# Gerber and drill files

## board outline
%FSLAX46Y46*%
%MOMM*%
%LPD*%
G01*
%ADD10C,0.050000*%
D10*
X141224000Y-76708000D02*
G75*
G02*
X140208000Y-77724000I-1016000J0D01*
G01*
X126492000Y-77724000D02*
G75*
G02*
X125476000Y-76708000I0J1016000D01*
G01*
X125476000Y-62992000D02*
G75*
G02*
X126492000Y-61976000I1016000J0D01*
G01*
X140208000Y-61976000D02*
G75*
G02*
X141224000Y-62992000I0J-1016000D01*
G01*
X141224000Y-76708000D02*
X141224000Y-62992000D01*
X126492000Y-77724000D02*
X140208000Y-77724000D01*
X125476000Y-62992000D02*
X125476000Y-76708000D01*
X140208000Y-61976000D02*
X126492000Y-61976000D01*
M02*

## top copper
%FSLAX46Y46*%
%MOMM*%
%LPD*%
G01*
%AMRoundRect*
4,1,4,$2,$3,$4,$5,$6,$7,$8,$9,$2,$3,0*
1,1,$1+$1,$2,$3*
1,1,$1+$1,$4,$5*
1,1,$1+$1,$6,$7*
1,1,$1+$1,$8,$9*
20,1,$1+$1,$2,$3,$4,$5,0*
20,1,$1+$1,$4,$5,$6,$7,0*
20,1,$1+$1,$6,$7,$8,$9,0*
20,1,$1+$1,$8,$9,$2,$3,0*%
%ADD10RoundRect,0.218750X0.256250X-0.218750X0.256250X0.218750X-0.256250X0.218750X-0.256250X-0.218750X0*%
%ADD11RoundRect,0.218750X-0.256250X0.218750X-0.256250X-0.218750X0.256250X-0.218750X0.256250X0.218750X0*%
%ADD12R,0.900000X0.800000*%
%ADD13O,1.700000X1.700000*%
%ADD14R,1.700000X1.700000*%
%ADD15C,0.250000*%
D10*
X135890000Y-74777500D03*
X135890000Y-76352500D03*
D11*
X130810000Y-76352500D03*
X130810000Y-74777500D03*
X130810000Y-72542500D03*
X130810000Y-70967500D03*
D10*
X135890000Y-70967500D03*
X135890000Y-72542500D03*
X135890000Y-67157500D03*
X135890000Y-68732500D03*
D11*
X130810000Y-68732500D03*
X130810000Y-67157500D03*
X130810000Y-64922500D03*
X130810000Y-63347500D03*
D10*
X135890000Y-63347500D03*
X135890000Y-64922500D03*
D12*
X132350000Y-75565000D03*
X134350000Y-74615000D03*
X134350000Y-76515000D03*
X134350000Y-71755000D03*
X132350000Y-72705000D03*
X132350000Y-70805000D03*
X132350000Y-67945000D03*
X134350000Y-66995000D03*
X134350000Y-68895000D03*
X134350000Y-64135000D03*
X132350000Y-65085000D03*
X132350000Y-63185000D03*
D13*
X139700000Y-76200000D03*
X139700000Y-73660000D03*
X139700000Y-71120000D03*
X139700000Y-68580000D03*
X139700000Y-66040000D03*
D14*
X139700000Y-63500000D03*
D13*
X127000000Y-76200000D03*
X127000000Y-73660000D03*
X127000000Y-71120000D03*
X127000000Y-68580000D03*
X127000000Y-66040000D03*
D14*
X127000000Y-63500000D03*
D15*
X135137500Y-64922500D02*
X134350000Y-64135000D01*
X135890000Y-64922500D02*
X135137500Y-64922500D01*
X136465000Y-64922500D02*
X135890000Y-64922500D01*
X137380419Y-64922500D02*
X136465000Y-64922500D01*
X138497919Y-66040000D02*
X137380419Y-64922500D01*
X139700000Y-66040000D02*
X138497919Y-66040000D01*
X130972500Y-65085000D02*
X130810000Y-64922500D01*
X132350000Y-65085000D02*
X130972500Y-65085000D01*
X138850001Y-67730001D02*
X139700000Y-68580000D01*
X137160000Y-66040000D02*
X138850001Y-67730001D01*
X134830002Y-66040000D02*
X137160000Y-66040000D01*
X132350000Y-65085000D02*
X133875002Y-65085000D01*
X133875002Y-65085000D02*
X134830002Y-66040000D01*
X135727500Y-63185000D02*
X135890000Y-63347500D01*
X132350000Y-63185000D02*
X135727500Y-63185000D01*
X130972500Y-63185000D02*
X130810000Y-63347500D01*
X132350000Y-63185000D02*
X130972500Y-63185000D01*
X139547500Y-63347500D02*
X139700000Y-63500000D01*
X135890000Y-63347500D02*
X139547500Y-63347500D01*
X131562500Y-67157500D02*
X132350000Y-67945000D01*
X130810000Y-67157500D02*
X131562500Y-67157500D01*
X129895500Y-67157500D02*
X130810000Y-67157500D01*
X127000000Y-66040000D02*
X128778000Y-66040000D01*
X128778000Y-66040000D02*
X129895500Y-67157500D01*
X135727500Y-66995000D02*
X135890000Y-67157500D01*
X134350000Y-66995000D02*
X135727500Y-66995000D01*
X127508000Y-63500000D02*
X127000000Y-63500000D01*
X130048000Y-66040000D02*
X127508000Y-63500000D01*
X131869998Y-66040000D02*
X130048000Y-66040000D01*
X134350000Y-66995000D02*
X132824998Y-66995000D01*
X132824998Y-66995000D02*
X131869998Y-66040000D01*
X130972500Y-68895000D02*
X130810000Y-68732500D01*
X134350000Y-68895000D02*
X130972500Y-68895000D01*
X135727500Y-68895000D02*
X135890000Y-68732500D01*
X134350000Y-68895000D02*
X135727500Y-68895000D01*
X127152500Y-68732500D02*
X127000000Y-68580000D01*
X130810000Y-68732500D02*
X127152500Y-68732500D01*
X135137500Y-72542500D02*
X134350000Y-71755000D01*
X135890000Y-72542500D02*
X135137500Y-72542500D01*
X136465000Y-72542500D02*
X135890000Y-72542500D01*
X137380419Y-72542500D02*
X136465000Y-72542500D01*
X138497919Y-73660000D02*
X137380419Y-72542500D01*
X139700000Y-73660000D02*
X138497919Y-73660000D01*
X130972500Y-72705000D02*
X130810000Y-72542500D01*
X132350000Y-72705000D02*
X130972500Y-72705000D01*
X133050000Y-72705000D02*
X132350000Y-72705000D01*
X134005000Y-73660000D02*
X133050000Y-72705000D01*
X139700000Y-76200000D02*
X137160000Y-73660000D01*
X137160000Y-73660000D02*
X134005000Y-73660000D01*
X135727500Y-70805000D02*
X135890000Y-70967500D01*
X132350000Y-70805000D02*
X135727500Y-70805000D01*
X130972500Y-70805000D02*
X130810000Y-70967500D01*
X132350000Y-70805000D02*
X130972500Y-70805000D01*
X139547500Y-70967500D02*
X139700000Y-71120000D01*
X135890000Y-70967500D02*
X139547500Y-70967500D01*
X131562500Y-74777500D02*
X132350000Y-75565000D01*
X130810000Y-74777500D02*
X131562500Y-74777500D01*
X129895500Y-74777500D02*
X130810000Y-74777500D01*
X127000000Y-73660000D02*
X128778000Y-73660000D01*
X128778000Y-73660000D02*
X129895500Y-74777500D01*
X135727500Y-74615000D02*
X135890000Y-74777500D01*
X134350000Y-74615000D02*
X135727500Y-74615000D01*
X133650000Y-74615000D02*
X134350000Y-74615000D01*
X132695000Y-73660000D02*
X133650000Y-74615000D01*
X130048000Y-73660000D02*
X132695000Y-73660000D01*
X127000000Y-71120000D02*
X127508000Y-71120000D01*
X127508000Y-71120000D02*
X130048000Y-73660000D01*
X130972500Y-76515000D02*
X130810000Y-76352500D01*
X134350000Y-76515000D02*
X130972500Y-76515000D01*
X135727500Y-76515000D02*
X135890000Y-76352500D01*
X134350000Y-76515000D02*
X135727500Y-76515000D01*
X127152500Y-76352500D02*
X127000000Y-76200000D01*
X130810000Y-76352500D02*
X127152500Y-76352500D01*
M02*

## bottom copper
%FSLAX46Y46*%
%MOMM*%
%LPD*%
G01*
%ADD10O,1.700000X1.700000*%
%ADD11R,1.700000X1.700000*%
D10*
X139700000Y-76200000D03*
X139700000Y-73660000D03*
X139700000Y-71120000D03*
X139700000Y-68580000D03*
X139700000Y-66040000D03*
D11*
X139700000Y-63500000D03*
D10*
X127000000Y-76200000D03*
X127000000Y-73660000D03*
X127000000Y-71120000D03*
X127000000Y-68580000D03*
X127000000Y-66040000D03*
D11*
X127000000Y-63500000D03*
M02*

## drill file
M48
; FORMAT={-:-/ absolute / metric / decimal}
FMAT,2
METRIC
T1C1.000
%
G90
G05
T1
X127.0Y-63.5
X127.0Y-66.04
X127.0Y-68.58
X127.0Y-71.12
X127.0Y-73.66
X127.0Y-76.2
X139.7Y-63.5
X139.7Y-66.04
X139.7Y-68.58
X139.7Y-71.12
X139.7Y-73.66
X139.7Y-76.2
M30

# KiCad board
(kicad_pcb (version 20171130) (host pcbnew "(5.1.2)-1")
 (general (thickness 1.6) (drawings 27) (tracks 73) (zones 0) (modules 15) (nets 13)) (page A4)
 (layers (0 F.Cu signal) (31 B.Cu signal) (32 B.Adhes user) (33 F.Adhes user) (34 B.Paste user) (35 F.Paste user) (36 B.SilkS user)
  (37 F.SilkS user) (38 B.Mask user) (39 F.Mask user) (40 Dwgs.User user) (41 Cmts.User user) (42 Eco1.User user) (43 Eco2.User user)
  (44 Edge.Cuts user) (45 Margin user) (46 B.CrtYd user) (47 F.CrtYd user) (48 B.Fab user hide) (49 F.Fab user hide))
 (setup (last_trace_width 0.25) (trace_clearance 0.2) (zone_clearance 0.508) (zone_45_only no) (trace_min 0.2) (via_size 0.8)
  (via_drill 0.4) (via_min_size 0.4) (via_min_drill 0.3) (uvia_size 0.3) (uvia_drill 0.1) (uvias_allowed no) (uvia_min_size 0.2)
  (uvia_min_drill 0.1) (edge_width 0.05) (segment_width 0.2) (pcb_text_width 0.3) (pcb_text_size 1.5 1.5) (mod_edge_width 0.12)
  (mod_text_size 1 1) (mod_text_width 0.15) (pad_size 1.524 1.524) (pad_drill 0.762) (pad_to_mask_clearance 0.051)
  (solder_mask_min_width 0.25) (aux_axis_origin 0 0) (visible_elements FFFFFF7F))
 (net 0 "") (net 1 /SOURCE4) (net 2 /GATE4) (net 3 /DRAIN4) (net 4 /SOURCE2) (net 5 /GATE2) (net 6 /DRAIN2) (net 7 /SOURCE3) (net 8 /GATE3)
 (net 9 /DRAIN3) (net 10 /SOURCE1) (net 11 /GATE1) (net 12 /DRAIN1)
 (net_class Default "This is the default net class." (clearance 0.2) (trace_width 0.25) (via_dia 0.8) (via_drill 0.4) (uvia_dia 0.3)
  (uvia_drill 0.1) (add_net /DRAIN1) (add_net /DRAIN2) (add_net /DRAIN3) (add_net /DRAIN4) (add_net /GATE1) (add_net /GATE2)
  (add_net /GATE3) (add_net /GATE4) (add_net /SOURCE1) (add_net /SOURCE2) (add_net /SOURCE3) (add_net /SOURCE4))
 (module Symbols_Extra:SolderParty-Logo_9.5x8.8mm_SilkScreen (layer B.Cu) (at 133.35 73.406 180)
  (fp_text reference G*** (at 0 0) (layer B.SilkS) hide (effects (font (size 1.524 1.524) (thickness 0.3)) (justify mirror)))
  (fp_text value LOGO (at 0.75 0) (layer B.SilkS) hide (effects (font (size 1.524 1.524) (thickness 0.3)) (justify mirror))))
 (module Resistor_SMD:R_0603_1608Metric (layer F.Cu) (at 135.89 75.565 90)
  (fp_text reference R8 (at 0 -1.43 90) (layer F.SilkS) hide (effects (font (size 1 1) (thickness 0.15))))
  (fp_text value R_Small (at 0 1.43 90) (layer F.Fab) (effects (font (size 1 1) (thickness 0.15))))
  (pad 2 smd roundrect (at 0.7875 0 90) (size 0.875 0.95) (layers F.Cu F.Paste F.Mask) (roundrect_rratio 0.25) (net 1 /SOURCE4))
  (pad 1 smd roundrect (at -0.7875 0 90) (size 0.875 0.95) (layers F.Cu F.Paste F.Mask) (roundrect_rratio 0.25) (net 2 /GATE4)))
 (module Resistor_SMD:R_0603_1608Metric (layer F.Cu) (at 130.81 75.565 270)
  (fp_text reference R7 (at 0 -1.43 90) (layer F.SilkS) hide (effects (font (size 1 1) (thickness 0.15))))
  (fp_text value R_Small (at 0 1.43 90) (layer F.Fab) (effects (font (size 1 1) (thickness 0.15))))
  (pad 2 smd roundrect (at 0.7875 0 270) (size 0.875 0.95) (layers F.Cu F.Paste F.Mask) (roundrect_rratio 0.25) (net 2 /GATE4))
  (pad 1 smd roundrect (at -0.7875 0 270) (size 0.875 0.95) (layers F.Cu F.Paste F.Mask) (roundrect_rratio 0.25) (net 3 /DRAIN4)))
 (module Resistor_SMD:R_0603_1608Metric (layer F.Cu) (at 130.81 71.755 270)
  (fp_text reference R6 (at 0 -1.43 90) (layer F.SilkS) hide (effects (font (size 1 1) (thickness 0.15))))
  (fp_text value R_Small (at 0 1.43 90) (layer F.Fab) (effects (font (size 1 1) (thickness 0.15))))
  (pad 2 smd roundrect (at 0.7875 0 270) (size 0.875 0.95) (layers F.Cu F.Paste F.Mask) (roundrect_rratio 0.25) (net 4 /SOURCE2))
  (pad 1 smd roundrect (at -0.7875 0 270) (size 0.875 0.95) (layers F.Cu F.Paste F.Mask) (roundrect_rratio 0.25) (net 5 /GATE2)))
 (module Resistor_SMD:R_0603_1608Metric (layer F.Cu) (at 135.89 71.755 90)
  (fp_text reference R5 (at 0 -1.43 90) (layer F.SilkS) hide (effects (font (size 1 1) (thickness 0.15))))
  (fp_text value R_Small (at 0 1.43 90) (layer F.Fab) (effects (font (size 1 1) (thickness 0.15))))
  (pad 2 smd roundrect (at 0.7875 0 90) (size 0.875 0.95) (layers F.Cu F.Paste F.Mask) (roundrect_rratio 0.25) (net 5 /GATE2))
  (pad 1 smd roundrect (at -0.7875 0 90) (size 0.875 0.95) (layers F.Cu F.Paste F.Mask) (roundrect_rratio 0.25) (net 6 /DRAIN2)))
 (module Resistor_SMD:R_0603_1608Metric (layer F.Cu) (at 135.89 67.945 90)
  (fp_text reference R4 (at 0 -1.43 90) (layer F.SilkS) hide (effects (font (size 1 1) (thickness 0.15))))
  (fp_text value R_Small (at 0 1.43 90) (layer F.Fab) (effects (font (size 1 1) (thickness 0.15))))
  (pad 2 smd roundrect (at 0.7875 0 90) (size 0.875 0.95) (layers F.Cu F.Paste F.Mask) (roundrect_rratio 0.25) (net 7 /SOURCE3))
  (pad 1 smd roundrect (at -0.7875 0 90) (size 0.875 0.95) (layers F.Cu F.Paste F.Mask) (roundrect_rratio 0.25) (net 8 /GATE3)))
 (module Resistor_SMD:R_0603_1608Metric (layer F.Cu) (at 130.81 67.945 270)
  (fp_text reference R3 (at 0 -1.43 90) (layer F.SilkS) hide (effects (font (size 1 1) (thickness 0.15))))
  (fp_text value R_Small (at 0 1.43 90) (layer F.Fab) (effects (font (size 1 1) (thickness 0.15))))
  (pad 2 smd roundrect (at 0.7875 0 270) (size 0.875 0.95) (layers F.Cu F.Paste F.Mask) (roundrect_rratio 0.25) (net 8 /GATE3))
  (pad 1 smd roundrect (at -0.7875 0 270) (size 0.875 0.95) (layers F.Cu F.Paste F.Mask) (roundrect_rratio 0.25) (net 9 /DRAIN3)))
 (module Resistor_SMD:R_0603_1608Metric (layer F.Cu) (at 130.81 64.135 270)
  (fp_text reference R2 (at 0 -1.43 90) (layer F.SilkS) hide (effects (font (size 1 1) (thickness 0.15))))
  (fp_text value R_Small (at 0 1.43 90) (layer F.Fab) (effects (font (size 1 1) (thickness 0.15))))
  (pad 2 smd roundrect (at 0.7875 0 270) (size 0.875 0.95) (layers F.Cu F.Paste F.Mask) (roundrect_rratio 0.25) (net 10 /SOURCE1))
  (pad 1 smd roundrect (at -0.7875 0 270) (size 0.875 0.95) (layers F.Cu F.Paste F.Mask) (roundrect_rratio 0.25) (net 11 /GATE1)))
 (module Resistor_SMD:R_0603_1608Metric (layer F.Cu) (at 135.89 64.135 90)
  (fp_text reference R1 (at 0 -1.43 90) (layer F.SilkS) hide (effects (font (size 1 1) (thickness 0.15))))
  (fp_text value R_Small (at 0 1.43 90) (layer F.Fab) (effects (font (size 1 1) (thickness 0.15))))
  (pad 2 smd roundrect (at 0.7875 0 90) (size 0.875 0.95) (layers F.Cu F.Paste F.Mask) (roundrect_rratio 0.25) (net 11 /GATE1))
  (pad 1 smd roundrect (at -0.7875 0 90) (size 0.875 0.95) (layers F.Cu F.Paste F.Mask) (roundrect_rratio 0.25) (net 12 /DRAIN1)))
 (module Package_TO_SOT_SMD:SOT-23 (layer F.Cu) (at 133.35 75.565 180)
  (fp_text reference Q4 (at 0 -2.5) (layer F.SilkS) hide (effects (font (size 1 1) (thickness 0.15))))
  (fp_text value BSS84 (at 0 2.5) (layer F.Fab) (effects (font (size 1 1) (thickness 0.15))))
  (pad 3 smd rect (at 1 0 180) (size 0.9 0.8) (layers F.Cu F.Paste F.Mask) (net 3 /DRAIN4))
  (pad 2 smd rect (at -1 0.95 180) (size 0.9 0.8) (layers F.Cu F.Paste F.Mask) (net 1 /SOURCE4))
  (pad 1 smd rect (at -1 -0.95 180) (size 0.9 0.8) (layers F.Cu F.Paste F.Mask) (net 2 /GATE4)))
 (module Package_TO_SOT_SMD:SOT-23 (layer F.Cu) (at 133.35 71.755)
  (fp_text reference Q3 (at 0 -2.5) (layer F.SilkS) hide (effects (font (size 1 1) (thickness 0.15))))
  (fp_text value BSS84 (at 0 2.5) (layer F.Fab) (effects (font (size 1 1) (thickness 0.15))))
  (pad 3 smd rect (at 1 0) (size 0.9 0.8) (layers F.Cu F.Paste F.Mask) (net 6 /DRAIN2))
  (pad 2 smd rect (at -1 0.95) (size 0.9 0.8) (layers F.Cu F.Paste F.Mask) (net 4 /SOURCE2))
  (pad 1 smd rect (at -1 -0.95) (size 0.9 0.8) (layers F.Cu F.Paste F.Mask) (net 5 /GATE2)))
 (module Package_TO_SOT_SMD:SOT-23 (layer F.Cu) (at 133.35 67.945 180)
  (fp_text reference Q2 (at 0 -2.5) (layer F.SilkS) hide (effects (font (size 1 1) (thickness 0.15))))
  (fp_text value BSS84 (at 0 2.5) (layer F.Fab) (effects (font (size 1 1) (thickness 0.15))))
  (pad 3 smd rect (at 1 0 180) (size 0.9 0.8) (layers F.Cu F.Paste F.Mask) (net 9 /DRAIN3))
  (pad 2 smd rect (at -1 0.95 180) (size 0.9 0.8) (layers F.Cu F.Paste F.Mask) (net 7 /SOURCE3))
  (pad 1 smd rect (at -1 -0.95 180) (size 0.9 0.8) (layers F.Cu F.Paste F.Mask) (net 8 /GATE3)))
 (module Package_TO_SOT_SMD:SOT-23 (layer F.Cu) (at 133.35 64.135)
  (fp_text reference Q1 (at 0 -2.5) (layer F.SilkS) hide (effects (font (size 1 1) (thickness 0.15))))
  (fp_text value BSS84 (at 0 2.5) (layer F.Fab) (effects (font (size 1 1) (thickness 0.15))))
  (pad 3 smd rect (at 1 0) (size 0.9 0.8) (layers F.Cu F.Paste F.Mask) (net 12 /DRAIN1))
  (pad 2 smd rect (at -1 0.95) (size 0.9 0.8) (layers F.Cu F.Paste F.Mask) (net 10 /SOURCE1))
  (pad 1 smd rect (at -1 -0.95) (size 0.9 0.8) (layers F.Cu F.Paste F.Mask) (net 11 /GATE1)))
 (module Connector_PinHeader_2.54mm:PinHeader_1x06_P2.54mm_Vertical (layer B.Cu) (at 139.7 63.5 180)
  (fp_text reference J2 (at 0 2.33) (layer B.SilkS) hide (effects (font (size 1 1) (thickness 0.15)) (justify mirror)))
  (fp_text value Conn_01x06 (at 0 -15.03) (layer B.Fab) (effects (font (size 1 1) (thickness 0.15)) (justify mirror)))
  (pad 6 thru_hole oval (at 0 -12.7 180) (size 1.7 1.7) (drill 1) (layers *.Cu *.Mask) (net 4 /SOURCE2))
  (pad 5 thru_hole oval (at 0 -10.16 180) (size 1.7 1.7) (drill 1) (layers *.Cu *.Mask) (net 6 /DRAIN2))
  (pad 4 thru_hole oval (at 0 -7.62 180) (size 1.7 1.7) (drill 1) (layers *.Cu *.Mask) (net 5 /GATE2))
  (pad 3 thru_hole oval (at 0 -5.08 180) (size 1.7 1.7) (drill 1) (layers *.Cu *.Mask) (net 10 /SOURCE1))
  (pad 2 thru_hole oval (at 0 -2.54 180) (size 1.7 1.7) (drill 1) (layers *.Cu *.Mask) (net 12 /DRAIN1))
  (pad 1 thru_hole rect (at 0 0 180) (size 1.7 1.7) (drill 1) (layers *.Cu *.Mask) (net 11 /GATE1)))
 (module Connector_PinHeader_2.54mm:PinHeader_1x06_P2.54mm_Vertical (layer B.Cu) (at 127 63.5 180)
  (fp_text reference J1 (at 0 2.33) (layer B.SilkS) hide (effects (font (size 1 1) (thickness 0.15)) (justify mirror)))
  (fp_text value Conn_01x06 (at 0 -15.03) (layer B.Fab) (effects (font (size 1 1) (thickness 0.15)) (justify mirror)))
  (pad 6 thru_hole oval (at 0 -12.7 180) (size 1.7 1.7) (drill 1) (layers *.Cu *.Mask) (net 2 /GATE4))
  (pad 5 thru_hole oval (at 0 -10.16 180) (size 1.7 1.7) (drill 1) (layers *.Cu *.Mask) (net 3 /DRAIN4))
  (pad 4 thru_hole oval (at 0 -7.62 180) (size 1.7 1.7) (drill 1) (layers *.Cu *.Mask) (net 1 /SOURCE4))
  (pad 3 thru_hole oval (at 0 -5.08 180) (size 1.7 1.7) (drill 1) (layers *.Cu *.Mask) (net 8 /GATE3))
  (pad 2 thru_hole oval (at 0 -2.54 180) (size 1.7 1.7) (drill 1) (layers *.Cu *.Mask) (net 9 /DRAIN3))
  (pad 1 thru_hole rect (at 0 0 180) (size 1.7 1.7) (drill 1) (layers *.Cu *.Mask) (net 7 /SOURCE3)))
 (gr_arc (start 140.208 76.708) (end 140.208 77.724) (angle -90) (layer Edge.Cuts) (width 0.05))
 (gr_arc (start 126.492 76.708) (end 125.476 76.708) (angle -90) (layer Edge.Cuts) (width 0.05))
 (gr_arc (start 126.492 62.992) (end 126.492 61.976) (angle -90) (layer Edge.Cuts) (width 0.05))
 (gr_arc (start 140.208 62.992) (end 141.224 62.992) (angle -90) (layer Edge.Cuts) (width 0.05))
 (gr_line (start 141.224 76.708) (end 141.224 62.992) (layer Edge.Cuts) (width 0.05))
 (gr_line (start 126.492 77.724) (end 140.208 77.724) (layer Edge.Cuts) (width 0.05))
 (gr_line (start 125.476 62.992) (end 125.476 76.708) (layer Edge.Cuts) (width 0.05))
 (gr_line (start 140.208 61.976) (end 126.492 61.976) (layer Edge.Cuts) (width 0.05))
 (segment (start 135.1375 64.9225) (end 134.35 64.135) (width 0.25) (layer F.Cu) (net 12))
 (segment (start 135.89 64.9225) (end 135.1375 64.9225) (width 0.25) (layer F.Cu) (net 12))
 (segment (start 136.465 64.9225) (end 135.89 64.9225) (width 0.25) (layer F.Cu) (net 12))
 (segment (start 137.380419 64.9225) (end 136.465 64.9225) (width 0.25) (layer F.Cu) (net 12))
 (segment (start 138.497919 66.04) (end 137.380419 64.9225) (width 0.25) (layer F.Cu) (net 12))
 (segment (start 139.7 66.04) (end 138.497919 66.04) (width 0.25) (layer F.Cu) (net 12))
 (segment (start 130.9725 65.085) (end 130.81 64.9225) (width 0.25) (layer F.Cu) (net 10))
 (segment (start 132.35 65.085) (end 130.9725 65.085) (width 0.25) (layer F.Cu) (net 10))
 (segment (start 138.850001 67.730001) (end 139.7 68.58) (width 0.25) (layer F.Cu) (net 10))
 (segment (start 137.16 66.04) (end 138.850001 67.730001) (width 0.25) (layer F.Cu) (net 10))
 (segment (start 134.830002 66.04) (end 137.16 66.04) (width 0.25) (layer F.Cu) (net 10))
 (segment (start 132.35 65.085) (end 133.875002 65.085) (width 0.25) (layer F.Cu) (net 10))
 (segment (start 133.875002 65.085) (end 134.830002 66.04) (width 0.25) (layer F.Cu) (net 10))
 (segment (start 135.7275 63.185) (end 135.89 63.3475) (width 0.25) (layer F.Cu) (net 11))
 (segment (start 132.35 63.185) (end 135.7275 63.185) (width 0.25) (layer F.Cu) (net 11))
 (segment (start 130.9725 63.185) (end 130.81 63.3475) (width 0.25) (layer F.Cu) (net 11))
 (segment (start 132.35 63.185) (end 130.9725 63.185) (width 0.25) (layer F.Cu) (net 11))
 (segment (start 139.5475 63.3475) (end 139.7 63.5) (width 0.25) (layer F.Cu) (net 11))
 (segment (start 135.89 63.3475) (end 139.5475 63.3475) (width 0.25) (layer F.Cu) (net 11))
 (segment (start 131.5625 67.1575) (end 132.35 67.945) (width 0.25) (layer F.Cu) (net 9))
 (segment (start 130.81 67.1575) (end 131.5625 67.1575) (width 0.25) (layer F.Cu) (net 9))
 (segment (start 129.8955 67.1575) (end 130.81 67.1575) (width 0.25) (layer F.Cu) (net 9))
 (segment (start 127 66.04) (end 128.778 66.04) (width 0.25) (layer F.Cu) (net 9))
 (segment (start 128.778 66.04) (end 129.8955 67.1575) (width 0.25) (layer F.Cu) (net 9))
 (segment (start 135.7275 66.995) (end 135.89 67.1575) (width 0.25) (layer F.Cu) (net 7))
 (segment (start 134.35 66.995) (end 135.7275 66.995) (width 0.25) (layer F.Cu) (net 7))
 (segment (start 127.508 63.5) (end 127 63.5) (width 0.25) (layer F.Cu) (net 7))
 (segment (start 130.048 66.04) (end 127.508 63.5) (width 0.25) (layer F.Cu) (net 7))
 (segment (start 131.869998 66.04) (end 130.048 66.04) (width 0.25) (layer F.Cu) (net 7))
 (segment (start 134.35 66.995) (end 132.824998 66.995) (width 0.25) (layer F.Cu) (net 7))
 (segment (start 132.824998 66.995) (end 131.869998 66.04) (width 0.25) (layer F.Cu) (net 7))
 (segment (start 130.9725 68.895) (end 130.81 68.7325) (width 0.25) (layer F.Cu) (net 8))
 (segment (start 134.35 68.895) (end 130.9725 68.895) (width 0.25) (layer F.Cu) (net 8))
 (segment (start 135.7275 68.895) (end 135.89 68.7325) (width 0.25) (layer F.Cu) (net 8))
 (segment (start 134.35 68.895) (end 135.7275 68.895) (width 0.25) (layer F.Cu) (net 8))
 (segment (start 127.1525 68.7325) (end 127 68.58) (width 0.25) (layer F.Cu) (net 8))
 (segment (start 130.81 68.7325) (end 127.1525 68.7325) (width 0.25) (layer F.Cu) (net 8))
 (segment (start 135.1375 72.5425) (end 134.35 71.755) (width 0.25) (layer F.Cu) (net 6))
 (segment (start 135.89 72.5425) (end 135.1375 72.5425) (width 0.25) (layer F.Cu) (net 6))
 (segment (start 136.465 72.5425) (end 135.89 72.5425) (width 0.25) (layer F.Cu) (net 6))
 (segment (start 137.380419 72.5425) (end 136.465 72.5425) (width 0.25) (layer F.Cu) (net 6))
 (segment (start 138.497919 73.66) (end 137.380419 72.5425) (width 0.25) (layer F.Cu) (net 6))
 (segment (start 139.7 73.66) (end 138.497919 73.66) (width 0.25) (layer F.Cu) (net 6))
 (segment (start 130.9725 72.705) (end 130.81 72.5425) (width 0.25) (layer F.Cu) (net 4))
 (segment (start 132.35 72.705) (end 130.9725 72.705) (width 0.25) (layer F.Cu) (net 4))
 (segment (start 133.05 72.705) (end 132.35 72.705) (width 0.25) (layer F.Cu) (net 4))
 (segment (start 134.005 73.66) (end 133.05 72.705) (width 0.25) (layer F.Cu) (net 4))
 (segment (start 139.7 76.2) (end 137.16 73.66) (width 0.25) (layer F.Cu) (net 4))
 (segment (start 137.16 73.66) (end 134.005 73.66) (width 0.25) (layer F.Cu) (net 4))
 (segment (start 135.7275 70.805) (end 135.89 70.9675) (width 0.25) (layer F.Cu) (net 5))
 (segment (start 132.35 70.805) (end 135.7275 70.805) (width 0.25) (layer F.Cu) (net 5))
 (segment (start 130.9725 70.805) (end 130.81 70.9675) (width 0.25) (layer F.Cu) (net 5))
 (segment (start 132.35 70.805) (end 130.9725 70.805) (width 0.25) (layer F.Cu) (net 5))
 (segment (start 139.5475 70.9675) (end 139.7 71.12) (width 0.25) (layer F.Cu) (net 5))
 (segment (start 135.89 70.9675) (end 139.5475 70.9675) (width 0.25) (layer F.Cu) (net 5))
 (segment (start 131.5625 74.7775) (end 132.35 75.565) (width 0.25) (layer F.Cu) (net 3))
 (segment (start 130.81 74.7775) (end 131.5625 74.7775) (width 0.25) (layer F.Cu) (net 3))
 (segment (start 129.8955 74.7775) (end 130.81 74.7775) (width 0.25) (layer F.Cu) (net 3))
 (segment (start 127 73.66) (end 128.778 73.66) (width 0.25) (layer F.Cu) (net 3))
 (segment (start 128.778 73.66) (end 129.8955 74.7775) (width 0.25) (layer F.Cu) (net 3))
 (segment (start 135.7275 74.615) (end 135.89 74.7775) (width 0.25) (layer F.Cu) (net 1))
 (segment (start 134.35 74.615) (end 135.7275 74.615) (width 0.25) (layer F.Cu) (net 1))
 (segment (start 133.65 74.615) (end 134.35 74.615) (width 0.25) (layer F.Cu) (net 1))
 (segment (start 132.695 73.66) (end 133.65 74.615) (width 0.25) (layer F.Cu) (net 1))
 (segment (start 130.048 73.66) (end 132.695 73.66) (width 0.25) (layer F.Cu) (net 1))
 (segment (start 127 71.12) (end 127.508 71.12) (width 0.25) (layer F.Cu) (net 1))
 (segment (start 127.508 71.12) (end 130.048 73.66) (width 0.25) (layer F.Cu) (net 1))
 (segment (start 130.9725 76.515) (end 130.81 76.3525) (width 0.25) (layer F.Cu) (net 2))
 (segment (start 134.35 76.515) (end 130.9725 76.515) (width 0.25) (layer F.Cu) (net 2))
 (segment (start 135.7275 76.515) (end 135.89 76.3525) (width 0.25) (layer F.Cu) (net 2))
 (segment (start 134.35 76.515) (end 135.7275 76.515) (width 0.25) (layer F.Cu) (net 2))
 (segment (start 127.1525 76.3525) (end 127 76.2) (width 0.25) (layer F.Cu) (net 2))
 (segment (start 130.81 76.3525) (end 127.1525 76.3525) (width 0.25) (layer F.Cu) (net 2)))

